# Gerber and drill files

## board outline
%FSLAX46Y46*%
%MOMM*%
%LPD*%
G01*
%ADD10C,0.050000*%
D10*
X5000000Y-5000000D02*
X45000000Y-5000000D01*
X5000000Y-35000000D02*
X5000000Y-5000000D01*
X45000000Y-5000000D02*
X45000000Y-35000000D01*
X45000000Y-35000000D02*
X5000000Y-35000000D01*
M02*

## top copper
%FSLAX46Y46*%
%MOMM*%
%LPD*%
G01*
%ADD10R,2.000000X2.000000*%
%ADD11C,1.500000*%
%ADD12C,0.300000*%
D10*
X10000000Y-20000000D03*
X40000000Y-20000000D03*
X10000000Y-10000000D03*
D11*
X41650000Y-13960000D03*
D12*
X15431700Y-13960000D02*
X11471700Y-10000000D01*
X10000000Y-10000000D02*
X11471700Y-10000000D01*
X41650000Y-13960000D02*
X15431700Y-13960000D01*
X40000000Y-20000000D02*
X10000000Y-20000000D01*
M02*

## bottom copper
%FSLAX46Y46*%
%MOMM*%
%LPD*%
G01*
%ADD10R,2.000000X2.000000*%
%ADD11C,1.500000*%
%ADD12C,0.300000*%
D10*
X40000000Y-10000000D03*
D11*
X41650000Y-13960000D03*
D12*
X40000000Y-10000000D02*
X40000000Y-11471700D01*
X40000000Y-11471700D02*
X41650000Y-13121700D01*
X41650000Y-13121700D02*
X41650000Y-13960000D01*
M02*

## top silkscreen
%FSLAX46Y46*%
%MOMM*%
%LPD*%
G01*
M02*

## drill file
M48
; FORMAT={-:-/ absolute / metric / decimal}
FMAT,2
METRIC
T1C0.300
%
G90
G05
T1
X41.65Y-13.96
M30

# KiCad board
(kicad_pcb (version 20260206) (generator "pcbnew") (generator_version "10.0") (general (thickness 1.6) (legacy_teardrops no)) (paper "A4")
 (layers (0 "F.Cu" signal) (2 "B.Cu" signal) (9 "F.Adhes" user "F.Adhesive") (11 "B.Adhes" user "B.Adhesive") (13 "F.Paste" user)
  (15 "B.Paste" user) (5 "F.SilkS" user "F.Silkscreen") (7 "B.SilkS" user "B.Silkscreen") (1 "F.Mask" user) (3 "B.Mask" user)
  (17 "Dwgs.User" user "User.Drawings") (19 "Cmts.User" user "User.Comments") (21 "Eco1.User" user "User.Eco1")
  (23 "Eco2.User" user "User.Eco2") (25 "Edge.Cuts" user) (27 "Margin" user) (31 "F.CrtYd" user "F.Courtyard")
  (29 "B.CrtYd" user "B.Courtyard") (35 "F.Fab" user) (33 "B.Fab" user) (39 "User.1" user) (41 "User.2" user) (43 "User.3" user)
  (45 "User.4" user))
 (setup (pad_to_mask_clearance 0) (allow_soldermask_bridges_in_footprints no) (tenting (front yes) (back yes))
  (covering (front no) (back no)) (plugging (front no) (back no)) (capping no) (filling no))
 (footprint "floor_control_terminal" (layer "F.Cu") (at 10 20)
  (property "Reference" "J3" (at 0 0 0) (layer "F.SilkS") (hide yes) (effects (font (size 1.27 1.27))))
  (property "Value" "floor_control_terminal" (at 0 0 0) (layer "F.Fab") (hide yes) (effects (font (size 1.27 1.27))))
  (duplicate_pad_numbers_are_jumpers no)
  (pad "1" smd rect (at 0 0) (size 2 2) (layers "F.Cu" "F.Mask" "F.Paste") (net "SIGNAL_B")))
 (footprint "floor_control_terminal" (layer "F.Cu") (at 40 20)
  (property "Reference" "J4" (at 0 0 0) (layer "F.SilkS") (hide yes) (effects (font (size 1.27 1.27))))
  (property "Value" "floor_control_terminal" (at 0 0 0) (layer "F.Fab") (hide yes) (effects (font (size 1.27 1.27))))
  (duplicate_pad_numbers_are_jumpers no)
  (pad "1" smd rect (at 0 0) (size 2 2) (layers "F.Cu" "F.Mask" "F.Paste") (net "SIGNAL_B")))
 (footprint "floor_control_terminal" (layer "F.Cu") (at 10 10)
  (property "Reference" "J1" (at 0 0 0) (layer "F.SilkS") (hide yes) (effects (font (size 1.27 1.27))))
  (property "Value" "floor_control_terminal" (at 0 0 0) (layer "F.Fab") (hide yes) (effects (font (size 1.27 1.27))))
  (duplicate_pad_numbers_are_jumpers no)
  (pad "1" smd rect (at 0 0) (size 2 2) (layers "F.Cu" "F.Mask" "F.Paste") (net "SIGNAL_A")))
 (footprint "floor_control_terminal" (layer "B.Cu") (at 40 10)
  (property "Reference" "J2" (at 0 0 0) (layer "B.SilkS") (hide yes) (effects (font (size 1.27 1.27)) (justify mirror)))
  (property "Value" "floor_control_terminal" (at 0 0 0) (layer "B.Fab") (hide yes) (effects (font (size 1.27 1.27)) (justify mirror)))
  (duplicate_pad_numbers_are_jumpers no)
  (pad "1" smd rect (at 0 0) (size 2 2) (layers "B.Cu" "B.Mask" "B.Paste") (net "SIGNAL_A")))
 (gr_line (start 5 5) (end 45 5) (stroke (width 0.05) (type default)) (layer "Edge.Cuts"))
 (gr_line (start 5 35) (end 5 5) (stroke (width 0.05) (type default)) (layer "Edge.Cuts"))
 (gr_line (start 45 5) (end 45 35) (stroke (width 0.05) (type default)) (layer "Edge.Cuts"))
 (gr_line (start 45 35) (end 5 35) (stroke (width 0.05) (type default)) (layer "Edge.Cuts"))
 (segment (start 15.4317 13.96) (end 11.4717 10) (width 0.3) (layer "F.Cu") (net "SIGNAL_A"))
 (segment (start 10 10) (end 11.4717 10) (width 0.3) (layer "F.Cu") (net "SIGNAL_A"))
 (segment (start 41.65 13.96) (end 15.4317 13.96) (width 0.3) (layer "F.Cu") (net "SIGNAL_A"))
 (via (at 41.65 13.96) (size 1.5) (drill 0.3) (layers "F.Cu" "B.Cu") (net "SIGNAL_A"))
 (segment (start 40 10) (end 40 11.4717) (width 0.3) (layer "B.Cu") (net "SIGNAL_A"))
 (segment (start 40 11.4717) (end 41.65 13.1217) (width 0.3) (layer "B.Cu") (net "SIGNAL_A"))
 (segment (start 41.65 13.1217) (end 41.65 13.96) (width 0.3) (layer "B.Cu") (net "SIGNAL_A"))
 (segment (start 40 20) (end 10 20) (width 0.3) (layer "F.Cu") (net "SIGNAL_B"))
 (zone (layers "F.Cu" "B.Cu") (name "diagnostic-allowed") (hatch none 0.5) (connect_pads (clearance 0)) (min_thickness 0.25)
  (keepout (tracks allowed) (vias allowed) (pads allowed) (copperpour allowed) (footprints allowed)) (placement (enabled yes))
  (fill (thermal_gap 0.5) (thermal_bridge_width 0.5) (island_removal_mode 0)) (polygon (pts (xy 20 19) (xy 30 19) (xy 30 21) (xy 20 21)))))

